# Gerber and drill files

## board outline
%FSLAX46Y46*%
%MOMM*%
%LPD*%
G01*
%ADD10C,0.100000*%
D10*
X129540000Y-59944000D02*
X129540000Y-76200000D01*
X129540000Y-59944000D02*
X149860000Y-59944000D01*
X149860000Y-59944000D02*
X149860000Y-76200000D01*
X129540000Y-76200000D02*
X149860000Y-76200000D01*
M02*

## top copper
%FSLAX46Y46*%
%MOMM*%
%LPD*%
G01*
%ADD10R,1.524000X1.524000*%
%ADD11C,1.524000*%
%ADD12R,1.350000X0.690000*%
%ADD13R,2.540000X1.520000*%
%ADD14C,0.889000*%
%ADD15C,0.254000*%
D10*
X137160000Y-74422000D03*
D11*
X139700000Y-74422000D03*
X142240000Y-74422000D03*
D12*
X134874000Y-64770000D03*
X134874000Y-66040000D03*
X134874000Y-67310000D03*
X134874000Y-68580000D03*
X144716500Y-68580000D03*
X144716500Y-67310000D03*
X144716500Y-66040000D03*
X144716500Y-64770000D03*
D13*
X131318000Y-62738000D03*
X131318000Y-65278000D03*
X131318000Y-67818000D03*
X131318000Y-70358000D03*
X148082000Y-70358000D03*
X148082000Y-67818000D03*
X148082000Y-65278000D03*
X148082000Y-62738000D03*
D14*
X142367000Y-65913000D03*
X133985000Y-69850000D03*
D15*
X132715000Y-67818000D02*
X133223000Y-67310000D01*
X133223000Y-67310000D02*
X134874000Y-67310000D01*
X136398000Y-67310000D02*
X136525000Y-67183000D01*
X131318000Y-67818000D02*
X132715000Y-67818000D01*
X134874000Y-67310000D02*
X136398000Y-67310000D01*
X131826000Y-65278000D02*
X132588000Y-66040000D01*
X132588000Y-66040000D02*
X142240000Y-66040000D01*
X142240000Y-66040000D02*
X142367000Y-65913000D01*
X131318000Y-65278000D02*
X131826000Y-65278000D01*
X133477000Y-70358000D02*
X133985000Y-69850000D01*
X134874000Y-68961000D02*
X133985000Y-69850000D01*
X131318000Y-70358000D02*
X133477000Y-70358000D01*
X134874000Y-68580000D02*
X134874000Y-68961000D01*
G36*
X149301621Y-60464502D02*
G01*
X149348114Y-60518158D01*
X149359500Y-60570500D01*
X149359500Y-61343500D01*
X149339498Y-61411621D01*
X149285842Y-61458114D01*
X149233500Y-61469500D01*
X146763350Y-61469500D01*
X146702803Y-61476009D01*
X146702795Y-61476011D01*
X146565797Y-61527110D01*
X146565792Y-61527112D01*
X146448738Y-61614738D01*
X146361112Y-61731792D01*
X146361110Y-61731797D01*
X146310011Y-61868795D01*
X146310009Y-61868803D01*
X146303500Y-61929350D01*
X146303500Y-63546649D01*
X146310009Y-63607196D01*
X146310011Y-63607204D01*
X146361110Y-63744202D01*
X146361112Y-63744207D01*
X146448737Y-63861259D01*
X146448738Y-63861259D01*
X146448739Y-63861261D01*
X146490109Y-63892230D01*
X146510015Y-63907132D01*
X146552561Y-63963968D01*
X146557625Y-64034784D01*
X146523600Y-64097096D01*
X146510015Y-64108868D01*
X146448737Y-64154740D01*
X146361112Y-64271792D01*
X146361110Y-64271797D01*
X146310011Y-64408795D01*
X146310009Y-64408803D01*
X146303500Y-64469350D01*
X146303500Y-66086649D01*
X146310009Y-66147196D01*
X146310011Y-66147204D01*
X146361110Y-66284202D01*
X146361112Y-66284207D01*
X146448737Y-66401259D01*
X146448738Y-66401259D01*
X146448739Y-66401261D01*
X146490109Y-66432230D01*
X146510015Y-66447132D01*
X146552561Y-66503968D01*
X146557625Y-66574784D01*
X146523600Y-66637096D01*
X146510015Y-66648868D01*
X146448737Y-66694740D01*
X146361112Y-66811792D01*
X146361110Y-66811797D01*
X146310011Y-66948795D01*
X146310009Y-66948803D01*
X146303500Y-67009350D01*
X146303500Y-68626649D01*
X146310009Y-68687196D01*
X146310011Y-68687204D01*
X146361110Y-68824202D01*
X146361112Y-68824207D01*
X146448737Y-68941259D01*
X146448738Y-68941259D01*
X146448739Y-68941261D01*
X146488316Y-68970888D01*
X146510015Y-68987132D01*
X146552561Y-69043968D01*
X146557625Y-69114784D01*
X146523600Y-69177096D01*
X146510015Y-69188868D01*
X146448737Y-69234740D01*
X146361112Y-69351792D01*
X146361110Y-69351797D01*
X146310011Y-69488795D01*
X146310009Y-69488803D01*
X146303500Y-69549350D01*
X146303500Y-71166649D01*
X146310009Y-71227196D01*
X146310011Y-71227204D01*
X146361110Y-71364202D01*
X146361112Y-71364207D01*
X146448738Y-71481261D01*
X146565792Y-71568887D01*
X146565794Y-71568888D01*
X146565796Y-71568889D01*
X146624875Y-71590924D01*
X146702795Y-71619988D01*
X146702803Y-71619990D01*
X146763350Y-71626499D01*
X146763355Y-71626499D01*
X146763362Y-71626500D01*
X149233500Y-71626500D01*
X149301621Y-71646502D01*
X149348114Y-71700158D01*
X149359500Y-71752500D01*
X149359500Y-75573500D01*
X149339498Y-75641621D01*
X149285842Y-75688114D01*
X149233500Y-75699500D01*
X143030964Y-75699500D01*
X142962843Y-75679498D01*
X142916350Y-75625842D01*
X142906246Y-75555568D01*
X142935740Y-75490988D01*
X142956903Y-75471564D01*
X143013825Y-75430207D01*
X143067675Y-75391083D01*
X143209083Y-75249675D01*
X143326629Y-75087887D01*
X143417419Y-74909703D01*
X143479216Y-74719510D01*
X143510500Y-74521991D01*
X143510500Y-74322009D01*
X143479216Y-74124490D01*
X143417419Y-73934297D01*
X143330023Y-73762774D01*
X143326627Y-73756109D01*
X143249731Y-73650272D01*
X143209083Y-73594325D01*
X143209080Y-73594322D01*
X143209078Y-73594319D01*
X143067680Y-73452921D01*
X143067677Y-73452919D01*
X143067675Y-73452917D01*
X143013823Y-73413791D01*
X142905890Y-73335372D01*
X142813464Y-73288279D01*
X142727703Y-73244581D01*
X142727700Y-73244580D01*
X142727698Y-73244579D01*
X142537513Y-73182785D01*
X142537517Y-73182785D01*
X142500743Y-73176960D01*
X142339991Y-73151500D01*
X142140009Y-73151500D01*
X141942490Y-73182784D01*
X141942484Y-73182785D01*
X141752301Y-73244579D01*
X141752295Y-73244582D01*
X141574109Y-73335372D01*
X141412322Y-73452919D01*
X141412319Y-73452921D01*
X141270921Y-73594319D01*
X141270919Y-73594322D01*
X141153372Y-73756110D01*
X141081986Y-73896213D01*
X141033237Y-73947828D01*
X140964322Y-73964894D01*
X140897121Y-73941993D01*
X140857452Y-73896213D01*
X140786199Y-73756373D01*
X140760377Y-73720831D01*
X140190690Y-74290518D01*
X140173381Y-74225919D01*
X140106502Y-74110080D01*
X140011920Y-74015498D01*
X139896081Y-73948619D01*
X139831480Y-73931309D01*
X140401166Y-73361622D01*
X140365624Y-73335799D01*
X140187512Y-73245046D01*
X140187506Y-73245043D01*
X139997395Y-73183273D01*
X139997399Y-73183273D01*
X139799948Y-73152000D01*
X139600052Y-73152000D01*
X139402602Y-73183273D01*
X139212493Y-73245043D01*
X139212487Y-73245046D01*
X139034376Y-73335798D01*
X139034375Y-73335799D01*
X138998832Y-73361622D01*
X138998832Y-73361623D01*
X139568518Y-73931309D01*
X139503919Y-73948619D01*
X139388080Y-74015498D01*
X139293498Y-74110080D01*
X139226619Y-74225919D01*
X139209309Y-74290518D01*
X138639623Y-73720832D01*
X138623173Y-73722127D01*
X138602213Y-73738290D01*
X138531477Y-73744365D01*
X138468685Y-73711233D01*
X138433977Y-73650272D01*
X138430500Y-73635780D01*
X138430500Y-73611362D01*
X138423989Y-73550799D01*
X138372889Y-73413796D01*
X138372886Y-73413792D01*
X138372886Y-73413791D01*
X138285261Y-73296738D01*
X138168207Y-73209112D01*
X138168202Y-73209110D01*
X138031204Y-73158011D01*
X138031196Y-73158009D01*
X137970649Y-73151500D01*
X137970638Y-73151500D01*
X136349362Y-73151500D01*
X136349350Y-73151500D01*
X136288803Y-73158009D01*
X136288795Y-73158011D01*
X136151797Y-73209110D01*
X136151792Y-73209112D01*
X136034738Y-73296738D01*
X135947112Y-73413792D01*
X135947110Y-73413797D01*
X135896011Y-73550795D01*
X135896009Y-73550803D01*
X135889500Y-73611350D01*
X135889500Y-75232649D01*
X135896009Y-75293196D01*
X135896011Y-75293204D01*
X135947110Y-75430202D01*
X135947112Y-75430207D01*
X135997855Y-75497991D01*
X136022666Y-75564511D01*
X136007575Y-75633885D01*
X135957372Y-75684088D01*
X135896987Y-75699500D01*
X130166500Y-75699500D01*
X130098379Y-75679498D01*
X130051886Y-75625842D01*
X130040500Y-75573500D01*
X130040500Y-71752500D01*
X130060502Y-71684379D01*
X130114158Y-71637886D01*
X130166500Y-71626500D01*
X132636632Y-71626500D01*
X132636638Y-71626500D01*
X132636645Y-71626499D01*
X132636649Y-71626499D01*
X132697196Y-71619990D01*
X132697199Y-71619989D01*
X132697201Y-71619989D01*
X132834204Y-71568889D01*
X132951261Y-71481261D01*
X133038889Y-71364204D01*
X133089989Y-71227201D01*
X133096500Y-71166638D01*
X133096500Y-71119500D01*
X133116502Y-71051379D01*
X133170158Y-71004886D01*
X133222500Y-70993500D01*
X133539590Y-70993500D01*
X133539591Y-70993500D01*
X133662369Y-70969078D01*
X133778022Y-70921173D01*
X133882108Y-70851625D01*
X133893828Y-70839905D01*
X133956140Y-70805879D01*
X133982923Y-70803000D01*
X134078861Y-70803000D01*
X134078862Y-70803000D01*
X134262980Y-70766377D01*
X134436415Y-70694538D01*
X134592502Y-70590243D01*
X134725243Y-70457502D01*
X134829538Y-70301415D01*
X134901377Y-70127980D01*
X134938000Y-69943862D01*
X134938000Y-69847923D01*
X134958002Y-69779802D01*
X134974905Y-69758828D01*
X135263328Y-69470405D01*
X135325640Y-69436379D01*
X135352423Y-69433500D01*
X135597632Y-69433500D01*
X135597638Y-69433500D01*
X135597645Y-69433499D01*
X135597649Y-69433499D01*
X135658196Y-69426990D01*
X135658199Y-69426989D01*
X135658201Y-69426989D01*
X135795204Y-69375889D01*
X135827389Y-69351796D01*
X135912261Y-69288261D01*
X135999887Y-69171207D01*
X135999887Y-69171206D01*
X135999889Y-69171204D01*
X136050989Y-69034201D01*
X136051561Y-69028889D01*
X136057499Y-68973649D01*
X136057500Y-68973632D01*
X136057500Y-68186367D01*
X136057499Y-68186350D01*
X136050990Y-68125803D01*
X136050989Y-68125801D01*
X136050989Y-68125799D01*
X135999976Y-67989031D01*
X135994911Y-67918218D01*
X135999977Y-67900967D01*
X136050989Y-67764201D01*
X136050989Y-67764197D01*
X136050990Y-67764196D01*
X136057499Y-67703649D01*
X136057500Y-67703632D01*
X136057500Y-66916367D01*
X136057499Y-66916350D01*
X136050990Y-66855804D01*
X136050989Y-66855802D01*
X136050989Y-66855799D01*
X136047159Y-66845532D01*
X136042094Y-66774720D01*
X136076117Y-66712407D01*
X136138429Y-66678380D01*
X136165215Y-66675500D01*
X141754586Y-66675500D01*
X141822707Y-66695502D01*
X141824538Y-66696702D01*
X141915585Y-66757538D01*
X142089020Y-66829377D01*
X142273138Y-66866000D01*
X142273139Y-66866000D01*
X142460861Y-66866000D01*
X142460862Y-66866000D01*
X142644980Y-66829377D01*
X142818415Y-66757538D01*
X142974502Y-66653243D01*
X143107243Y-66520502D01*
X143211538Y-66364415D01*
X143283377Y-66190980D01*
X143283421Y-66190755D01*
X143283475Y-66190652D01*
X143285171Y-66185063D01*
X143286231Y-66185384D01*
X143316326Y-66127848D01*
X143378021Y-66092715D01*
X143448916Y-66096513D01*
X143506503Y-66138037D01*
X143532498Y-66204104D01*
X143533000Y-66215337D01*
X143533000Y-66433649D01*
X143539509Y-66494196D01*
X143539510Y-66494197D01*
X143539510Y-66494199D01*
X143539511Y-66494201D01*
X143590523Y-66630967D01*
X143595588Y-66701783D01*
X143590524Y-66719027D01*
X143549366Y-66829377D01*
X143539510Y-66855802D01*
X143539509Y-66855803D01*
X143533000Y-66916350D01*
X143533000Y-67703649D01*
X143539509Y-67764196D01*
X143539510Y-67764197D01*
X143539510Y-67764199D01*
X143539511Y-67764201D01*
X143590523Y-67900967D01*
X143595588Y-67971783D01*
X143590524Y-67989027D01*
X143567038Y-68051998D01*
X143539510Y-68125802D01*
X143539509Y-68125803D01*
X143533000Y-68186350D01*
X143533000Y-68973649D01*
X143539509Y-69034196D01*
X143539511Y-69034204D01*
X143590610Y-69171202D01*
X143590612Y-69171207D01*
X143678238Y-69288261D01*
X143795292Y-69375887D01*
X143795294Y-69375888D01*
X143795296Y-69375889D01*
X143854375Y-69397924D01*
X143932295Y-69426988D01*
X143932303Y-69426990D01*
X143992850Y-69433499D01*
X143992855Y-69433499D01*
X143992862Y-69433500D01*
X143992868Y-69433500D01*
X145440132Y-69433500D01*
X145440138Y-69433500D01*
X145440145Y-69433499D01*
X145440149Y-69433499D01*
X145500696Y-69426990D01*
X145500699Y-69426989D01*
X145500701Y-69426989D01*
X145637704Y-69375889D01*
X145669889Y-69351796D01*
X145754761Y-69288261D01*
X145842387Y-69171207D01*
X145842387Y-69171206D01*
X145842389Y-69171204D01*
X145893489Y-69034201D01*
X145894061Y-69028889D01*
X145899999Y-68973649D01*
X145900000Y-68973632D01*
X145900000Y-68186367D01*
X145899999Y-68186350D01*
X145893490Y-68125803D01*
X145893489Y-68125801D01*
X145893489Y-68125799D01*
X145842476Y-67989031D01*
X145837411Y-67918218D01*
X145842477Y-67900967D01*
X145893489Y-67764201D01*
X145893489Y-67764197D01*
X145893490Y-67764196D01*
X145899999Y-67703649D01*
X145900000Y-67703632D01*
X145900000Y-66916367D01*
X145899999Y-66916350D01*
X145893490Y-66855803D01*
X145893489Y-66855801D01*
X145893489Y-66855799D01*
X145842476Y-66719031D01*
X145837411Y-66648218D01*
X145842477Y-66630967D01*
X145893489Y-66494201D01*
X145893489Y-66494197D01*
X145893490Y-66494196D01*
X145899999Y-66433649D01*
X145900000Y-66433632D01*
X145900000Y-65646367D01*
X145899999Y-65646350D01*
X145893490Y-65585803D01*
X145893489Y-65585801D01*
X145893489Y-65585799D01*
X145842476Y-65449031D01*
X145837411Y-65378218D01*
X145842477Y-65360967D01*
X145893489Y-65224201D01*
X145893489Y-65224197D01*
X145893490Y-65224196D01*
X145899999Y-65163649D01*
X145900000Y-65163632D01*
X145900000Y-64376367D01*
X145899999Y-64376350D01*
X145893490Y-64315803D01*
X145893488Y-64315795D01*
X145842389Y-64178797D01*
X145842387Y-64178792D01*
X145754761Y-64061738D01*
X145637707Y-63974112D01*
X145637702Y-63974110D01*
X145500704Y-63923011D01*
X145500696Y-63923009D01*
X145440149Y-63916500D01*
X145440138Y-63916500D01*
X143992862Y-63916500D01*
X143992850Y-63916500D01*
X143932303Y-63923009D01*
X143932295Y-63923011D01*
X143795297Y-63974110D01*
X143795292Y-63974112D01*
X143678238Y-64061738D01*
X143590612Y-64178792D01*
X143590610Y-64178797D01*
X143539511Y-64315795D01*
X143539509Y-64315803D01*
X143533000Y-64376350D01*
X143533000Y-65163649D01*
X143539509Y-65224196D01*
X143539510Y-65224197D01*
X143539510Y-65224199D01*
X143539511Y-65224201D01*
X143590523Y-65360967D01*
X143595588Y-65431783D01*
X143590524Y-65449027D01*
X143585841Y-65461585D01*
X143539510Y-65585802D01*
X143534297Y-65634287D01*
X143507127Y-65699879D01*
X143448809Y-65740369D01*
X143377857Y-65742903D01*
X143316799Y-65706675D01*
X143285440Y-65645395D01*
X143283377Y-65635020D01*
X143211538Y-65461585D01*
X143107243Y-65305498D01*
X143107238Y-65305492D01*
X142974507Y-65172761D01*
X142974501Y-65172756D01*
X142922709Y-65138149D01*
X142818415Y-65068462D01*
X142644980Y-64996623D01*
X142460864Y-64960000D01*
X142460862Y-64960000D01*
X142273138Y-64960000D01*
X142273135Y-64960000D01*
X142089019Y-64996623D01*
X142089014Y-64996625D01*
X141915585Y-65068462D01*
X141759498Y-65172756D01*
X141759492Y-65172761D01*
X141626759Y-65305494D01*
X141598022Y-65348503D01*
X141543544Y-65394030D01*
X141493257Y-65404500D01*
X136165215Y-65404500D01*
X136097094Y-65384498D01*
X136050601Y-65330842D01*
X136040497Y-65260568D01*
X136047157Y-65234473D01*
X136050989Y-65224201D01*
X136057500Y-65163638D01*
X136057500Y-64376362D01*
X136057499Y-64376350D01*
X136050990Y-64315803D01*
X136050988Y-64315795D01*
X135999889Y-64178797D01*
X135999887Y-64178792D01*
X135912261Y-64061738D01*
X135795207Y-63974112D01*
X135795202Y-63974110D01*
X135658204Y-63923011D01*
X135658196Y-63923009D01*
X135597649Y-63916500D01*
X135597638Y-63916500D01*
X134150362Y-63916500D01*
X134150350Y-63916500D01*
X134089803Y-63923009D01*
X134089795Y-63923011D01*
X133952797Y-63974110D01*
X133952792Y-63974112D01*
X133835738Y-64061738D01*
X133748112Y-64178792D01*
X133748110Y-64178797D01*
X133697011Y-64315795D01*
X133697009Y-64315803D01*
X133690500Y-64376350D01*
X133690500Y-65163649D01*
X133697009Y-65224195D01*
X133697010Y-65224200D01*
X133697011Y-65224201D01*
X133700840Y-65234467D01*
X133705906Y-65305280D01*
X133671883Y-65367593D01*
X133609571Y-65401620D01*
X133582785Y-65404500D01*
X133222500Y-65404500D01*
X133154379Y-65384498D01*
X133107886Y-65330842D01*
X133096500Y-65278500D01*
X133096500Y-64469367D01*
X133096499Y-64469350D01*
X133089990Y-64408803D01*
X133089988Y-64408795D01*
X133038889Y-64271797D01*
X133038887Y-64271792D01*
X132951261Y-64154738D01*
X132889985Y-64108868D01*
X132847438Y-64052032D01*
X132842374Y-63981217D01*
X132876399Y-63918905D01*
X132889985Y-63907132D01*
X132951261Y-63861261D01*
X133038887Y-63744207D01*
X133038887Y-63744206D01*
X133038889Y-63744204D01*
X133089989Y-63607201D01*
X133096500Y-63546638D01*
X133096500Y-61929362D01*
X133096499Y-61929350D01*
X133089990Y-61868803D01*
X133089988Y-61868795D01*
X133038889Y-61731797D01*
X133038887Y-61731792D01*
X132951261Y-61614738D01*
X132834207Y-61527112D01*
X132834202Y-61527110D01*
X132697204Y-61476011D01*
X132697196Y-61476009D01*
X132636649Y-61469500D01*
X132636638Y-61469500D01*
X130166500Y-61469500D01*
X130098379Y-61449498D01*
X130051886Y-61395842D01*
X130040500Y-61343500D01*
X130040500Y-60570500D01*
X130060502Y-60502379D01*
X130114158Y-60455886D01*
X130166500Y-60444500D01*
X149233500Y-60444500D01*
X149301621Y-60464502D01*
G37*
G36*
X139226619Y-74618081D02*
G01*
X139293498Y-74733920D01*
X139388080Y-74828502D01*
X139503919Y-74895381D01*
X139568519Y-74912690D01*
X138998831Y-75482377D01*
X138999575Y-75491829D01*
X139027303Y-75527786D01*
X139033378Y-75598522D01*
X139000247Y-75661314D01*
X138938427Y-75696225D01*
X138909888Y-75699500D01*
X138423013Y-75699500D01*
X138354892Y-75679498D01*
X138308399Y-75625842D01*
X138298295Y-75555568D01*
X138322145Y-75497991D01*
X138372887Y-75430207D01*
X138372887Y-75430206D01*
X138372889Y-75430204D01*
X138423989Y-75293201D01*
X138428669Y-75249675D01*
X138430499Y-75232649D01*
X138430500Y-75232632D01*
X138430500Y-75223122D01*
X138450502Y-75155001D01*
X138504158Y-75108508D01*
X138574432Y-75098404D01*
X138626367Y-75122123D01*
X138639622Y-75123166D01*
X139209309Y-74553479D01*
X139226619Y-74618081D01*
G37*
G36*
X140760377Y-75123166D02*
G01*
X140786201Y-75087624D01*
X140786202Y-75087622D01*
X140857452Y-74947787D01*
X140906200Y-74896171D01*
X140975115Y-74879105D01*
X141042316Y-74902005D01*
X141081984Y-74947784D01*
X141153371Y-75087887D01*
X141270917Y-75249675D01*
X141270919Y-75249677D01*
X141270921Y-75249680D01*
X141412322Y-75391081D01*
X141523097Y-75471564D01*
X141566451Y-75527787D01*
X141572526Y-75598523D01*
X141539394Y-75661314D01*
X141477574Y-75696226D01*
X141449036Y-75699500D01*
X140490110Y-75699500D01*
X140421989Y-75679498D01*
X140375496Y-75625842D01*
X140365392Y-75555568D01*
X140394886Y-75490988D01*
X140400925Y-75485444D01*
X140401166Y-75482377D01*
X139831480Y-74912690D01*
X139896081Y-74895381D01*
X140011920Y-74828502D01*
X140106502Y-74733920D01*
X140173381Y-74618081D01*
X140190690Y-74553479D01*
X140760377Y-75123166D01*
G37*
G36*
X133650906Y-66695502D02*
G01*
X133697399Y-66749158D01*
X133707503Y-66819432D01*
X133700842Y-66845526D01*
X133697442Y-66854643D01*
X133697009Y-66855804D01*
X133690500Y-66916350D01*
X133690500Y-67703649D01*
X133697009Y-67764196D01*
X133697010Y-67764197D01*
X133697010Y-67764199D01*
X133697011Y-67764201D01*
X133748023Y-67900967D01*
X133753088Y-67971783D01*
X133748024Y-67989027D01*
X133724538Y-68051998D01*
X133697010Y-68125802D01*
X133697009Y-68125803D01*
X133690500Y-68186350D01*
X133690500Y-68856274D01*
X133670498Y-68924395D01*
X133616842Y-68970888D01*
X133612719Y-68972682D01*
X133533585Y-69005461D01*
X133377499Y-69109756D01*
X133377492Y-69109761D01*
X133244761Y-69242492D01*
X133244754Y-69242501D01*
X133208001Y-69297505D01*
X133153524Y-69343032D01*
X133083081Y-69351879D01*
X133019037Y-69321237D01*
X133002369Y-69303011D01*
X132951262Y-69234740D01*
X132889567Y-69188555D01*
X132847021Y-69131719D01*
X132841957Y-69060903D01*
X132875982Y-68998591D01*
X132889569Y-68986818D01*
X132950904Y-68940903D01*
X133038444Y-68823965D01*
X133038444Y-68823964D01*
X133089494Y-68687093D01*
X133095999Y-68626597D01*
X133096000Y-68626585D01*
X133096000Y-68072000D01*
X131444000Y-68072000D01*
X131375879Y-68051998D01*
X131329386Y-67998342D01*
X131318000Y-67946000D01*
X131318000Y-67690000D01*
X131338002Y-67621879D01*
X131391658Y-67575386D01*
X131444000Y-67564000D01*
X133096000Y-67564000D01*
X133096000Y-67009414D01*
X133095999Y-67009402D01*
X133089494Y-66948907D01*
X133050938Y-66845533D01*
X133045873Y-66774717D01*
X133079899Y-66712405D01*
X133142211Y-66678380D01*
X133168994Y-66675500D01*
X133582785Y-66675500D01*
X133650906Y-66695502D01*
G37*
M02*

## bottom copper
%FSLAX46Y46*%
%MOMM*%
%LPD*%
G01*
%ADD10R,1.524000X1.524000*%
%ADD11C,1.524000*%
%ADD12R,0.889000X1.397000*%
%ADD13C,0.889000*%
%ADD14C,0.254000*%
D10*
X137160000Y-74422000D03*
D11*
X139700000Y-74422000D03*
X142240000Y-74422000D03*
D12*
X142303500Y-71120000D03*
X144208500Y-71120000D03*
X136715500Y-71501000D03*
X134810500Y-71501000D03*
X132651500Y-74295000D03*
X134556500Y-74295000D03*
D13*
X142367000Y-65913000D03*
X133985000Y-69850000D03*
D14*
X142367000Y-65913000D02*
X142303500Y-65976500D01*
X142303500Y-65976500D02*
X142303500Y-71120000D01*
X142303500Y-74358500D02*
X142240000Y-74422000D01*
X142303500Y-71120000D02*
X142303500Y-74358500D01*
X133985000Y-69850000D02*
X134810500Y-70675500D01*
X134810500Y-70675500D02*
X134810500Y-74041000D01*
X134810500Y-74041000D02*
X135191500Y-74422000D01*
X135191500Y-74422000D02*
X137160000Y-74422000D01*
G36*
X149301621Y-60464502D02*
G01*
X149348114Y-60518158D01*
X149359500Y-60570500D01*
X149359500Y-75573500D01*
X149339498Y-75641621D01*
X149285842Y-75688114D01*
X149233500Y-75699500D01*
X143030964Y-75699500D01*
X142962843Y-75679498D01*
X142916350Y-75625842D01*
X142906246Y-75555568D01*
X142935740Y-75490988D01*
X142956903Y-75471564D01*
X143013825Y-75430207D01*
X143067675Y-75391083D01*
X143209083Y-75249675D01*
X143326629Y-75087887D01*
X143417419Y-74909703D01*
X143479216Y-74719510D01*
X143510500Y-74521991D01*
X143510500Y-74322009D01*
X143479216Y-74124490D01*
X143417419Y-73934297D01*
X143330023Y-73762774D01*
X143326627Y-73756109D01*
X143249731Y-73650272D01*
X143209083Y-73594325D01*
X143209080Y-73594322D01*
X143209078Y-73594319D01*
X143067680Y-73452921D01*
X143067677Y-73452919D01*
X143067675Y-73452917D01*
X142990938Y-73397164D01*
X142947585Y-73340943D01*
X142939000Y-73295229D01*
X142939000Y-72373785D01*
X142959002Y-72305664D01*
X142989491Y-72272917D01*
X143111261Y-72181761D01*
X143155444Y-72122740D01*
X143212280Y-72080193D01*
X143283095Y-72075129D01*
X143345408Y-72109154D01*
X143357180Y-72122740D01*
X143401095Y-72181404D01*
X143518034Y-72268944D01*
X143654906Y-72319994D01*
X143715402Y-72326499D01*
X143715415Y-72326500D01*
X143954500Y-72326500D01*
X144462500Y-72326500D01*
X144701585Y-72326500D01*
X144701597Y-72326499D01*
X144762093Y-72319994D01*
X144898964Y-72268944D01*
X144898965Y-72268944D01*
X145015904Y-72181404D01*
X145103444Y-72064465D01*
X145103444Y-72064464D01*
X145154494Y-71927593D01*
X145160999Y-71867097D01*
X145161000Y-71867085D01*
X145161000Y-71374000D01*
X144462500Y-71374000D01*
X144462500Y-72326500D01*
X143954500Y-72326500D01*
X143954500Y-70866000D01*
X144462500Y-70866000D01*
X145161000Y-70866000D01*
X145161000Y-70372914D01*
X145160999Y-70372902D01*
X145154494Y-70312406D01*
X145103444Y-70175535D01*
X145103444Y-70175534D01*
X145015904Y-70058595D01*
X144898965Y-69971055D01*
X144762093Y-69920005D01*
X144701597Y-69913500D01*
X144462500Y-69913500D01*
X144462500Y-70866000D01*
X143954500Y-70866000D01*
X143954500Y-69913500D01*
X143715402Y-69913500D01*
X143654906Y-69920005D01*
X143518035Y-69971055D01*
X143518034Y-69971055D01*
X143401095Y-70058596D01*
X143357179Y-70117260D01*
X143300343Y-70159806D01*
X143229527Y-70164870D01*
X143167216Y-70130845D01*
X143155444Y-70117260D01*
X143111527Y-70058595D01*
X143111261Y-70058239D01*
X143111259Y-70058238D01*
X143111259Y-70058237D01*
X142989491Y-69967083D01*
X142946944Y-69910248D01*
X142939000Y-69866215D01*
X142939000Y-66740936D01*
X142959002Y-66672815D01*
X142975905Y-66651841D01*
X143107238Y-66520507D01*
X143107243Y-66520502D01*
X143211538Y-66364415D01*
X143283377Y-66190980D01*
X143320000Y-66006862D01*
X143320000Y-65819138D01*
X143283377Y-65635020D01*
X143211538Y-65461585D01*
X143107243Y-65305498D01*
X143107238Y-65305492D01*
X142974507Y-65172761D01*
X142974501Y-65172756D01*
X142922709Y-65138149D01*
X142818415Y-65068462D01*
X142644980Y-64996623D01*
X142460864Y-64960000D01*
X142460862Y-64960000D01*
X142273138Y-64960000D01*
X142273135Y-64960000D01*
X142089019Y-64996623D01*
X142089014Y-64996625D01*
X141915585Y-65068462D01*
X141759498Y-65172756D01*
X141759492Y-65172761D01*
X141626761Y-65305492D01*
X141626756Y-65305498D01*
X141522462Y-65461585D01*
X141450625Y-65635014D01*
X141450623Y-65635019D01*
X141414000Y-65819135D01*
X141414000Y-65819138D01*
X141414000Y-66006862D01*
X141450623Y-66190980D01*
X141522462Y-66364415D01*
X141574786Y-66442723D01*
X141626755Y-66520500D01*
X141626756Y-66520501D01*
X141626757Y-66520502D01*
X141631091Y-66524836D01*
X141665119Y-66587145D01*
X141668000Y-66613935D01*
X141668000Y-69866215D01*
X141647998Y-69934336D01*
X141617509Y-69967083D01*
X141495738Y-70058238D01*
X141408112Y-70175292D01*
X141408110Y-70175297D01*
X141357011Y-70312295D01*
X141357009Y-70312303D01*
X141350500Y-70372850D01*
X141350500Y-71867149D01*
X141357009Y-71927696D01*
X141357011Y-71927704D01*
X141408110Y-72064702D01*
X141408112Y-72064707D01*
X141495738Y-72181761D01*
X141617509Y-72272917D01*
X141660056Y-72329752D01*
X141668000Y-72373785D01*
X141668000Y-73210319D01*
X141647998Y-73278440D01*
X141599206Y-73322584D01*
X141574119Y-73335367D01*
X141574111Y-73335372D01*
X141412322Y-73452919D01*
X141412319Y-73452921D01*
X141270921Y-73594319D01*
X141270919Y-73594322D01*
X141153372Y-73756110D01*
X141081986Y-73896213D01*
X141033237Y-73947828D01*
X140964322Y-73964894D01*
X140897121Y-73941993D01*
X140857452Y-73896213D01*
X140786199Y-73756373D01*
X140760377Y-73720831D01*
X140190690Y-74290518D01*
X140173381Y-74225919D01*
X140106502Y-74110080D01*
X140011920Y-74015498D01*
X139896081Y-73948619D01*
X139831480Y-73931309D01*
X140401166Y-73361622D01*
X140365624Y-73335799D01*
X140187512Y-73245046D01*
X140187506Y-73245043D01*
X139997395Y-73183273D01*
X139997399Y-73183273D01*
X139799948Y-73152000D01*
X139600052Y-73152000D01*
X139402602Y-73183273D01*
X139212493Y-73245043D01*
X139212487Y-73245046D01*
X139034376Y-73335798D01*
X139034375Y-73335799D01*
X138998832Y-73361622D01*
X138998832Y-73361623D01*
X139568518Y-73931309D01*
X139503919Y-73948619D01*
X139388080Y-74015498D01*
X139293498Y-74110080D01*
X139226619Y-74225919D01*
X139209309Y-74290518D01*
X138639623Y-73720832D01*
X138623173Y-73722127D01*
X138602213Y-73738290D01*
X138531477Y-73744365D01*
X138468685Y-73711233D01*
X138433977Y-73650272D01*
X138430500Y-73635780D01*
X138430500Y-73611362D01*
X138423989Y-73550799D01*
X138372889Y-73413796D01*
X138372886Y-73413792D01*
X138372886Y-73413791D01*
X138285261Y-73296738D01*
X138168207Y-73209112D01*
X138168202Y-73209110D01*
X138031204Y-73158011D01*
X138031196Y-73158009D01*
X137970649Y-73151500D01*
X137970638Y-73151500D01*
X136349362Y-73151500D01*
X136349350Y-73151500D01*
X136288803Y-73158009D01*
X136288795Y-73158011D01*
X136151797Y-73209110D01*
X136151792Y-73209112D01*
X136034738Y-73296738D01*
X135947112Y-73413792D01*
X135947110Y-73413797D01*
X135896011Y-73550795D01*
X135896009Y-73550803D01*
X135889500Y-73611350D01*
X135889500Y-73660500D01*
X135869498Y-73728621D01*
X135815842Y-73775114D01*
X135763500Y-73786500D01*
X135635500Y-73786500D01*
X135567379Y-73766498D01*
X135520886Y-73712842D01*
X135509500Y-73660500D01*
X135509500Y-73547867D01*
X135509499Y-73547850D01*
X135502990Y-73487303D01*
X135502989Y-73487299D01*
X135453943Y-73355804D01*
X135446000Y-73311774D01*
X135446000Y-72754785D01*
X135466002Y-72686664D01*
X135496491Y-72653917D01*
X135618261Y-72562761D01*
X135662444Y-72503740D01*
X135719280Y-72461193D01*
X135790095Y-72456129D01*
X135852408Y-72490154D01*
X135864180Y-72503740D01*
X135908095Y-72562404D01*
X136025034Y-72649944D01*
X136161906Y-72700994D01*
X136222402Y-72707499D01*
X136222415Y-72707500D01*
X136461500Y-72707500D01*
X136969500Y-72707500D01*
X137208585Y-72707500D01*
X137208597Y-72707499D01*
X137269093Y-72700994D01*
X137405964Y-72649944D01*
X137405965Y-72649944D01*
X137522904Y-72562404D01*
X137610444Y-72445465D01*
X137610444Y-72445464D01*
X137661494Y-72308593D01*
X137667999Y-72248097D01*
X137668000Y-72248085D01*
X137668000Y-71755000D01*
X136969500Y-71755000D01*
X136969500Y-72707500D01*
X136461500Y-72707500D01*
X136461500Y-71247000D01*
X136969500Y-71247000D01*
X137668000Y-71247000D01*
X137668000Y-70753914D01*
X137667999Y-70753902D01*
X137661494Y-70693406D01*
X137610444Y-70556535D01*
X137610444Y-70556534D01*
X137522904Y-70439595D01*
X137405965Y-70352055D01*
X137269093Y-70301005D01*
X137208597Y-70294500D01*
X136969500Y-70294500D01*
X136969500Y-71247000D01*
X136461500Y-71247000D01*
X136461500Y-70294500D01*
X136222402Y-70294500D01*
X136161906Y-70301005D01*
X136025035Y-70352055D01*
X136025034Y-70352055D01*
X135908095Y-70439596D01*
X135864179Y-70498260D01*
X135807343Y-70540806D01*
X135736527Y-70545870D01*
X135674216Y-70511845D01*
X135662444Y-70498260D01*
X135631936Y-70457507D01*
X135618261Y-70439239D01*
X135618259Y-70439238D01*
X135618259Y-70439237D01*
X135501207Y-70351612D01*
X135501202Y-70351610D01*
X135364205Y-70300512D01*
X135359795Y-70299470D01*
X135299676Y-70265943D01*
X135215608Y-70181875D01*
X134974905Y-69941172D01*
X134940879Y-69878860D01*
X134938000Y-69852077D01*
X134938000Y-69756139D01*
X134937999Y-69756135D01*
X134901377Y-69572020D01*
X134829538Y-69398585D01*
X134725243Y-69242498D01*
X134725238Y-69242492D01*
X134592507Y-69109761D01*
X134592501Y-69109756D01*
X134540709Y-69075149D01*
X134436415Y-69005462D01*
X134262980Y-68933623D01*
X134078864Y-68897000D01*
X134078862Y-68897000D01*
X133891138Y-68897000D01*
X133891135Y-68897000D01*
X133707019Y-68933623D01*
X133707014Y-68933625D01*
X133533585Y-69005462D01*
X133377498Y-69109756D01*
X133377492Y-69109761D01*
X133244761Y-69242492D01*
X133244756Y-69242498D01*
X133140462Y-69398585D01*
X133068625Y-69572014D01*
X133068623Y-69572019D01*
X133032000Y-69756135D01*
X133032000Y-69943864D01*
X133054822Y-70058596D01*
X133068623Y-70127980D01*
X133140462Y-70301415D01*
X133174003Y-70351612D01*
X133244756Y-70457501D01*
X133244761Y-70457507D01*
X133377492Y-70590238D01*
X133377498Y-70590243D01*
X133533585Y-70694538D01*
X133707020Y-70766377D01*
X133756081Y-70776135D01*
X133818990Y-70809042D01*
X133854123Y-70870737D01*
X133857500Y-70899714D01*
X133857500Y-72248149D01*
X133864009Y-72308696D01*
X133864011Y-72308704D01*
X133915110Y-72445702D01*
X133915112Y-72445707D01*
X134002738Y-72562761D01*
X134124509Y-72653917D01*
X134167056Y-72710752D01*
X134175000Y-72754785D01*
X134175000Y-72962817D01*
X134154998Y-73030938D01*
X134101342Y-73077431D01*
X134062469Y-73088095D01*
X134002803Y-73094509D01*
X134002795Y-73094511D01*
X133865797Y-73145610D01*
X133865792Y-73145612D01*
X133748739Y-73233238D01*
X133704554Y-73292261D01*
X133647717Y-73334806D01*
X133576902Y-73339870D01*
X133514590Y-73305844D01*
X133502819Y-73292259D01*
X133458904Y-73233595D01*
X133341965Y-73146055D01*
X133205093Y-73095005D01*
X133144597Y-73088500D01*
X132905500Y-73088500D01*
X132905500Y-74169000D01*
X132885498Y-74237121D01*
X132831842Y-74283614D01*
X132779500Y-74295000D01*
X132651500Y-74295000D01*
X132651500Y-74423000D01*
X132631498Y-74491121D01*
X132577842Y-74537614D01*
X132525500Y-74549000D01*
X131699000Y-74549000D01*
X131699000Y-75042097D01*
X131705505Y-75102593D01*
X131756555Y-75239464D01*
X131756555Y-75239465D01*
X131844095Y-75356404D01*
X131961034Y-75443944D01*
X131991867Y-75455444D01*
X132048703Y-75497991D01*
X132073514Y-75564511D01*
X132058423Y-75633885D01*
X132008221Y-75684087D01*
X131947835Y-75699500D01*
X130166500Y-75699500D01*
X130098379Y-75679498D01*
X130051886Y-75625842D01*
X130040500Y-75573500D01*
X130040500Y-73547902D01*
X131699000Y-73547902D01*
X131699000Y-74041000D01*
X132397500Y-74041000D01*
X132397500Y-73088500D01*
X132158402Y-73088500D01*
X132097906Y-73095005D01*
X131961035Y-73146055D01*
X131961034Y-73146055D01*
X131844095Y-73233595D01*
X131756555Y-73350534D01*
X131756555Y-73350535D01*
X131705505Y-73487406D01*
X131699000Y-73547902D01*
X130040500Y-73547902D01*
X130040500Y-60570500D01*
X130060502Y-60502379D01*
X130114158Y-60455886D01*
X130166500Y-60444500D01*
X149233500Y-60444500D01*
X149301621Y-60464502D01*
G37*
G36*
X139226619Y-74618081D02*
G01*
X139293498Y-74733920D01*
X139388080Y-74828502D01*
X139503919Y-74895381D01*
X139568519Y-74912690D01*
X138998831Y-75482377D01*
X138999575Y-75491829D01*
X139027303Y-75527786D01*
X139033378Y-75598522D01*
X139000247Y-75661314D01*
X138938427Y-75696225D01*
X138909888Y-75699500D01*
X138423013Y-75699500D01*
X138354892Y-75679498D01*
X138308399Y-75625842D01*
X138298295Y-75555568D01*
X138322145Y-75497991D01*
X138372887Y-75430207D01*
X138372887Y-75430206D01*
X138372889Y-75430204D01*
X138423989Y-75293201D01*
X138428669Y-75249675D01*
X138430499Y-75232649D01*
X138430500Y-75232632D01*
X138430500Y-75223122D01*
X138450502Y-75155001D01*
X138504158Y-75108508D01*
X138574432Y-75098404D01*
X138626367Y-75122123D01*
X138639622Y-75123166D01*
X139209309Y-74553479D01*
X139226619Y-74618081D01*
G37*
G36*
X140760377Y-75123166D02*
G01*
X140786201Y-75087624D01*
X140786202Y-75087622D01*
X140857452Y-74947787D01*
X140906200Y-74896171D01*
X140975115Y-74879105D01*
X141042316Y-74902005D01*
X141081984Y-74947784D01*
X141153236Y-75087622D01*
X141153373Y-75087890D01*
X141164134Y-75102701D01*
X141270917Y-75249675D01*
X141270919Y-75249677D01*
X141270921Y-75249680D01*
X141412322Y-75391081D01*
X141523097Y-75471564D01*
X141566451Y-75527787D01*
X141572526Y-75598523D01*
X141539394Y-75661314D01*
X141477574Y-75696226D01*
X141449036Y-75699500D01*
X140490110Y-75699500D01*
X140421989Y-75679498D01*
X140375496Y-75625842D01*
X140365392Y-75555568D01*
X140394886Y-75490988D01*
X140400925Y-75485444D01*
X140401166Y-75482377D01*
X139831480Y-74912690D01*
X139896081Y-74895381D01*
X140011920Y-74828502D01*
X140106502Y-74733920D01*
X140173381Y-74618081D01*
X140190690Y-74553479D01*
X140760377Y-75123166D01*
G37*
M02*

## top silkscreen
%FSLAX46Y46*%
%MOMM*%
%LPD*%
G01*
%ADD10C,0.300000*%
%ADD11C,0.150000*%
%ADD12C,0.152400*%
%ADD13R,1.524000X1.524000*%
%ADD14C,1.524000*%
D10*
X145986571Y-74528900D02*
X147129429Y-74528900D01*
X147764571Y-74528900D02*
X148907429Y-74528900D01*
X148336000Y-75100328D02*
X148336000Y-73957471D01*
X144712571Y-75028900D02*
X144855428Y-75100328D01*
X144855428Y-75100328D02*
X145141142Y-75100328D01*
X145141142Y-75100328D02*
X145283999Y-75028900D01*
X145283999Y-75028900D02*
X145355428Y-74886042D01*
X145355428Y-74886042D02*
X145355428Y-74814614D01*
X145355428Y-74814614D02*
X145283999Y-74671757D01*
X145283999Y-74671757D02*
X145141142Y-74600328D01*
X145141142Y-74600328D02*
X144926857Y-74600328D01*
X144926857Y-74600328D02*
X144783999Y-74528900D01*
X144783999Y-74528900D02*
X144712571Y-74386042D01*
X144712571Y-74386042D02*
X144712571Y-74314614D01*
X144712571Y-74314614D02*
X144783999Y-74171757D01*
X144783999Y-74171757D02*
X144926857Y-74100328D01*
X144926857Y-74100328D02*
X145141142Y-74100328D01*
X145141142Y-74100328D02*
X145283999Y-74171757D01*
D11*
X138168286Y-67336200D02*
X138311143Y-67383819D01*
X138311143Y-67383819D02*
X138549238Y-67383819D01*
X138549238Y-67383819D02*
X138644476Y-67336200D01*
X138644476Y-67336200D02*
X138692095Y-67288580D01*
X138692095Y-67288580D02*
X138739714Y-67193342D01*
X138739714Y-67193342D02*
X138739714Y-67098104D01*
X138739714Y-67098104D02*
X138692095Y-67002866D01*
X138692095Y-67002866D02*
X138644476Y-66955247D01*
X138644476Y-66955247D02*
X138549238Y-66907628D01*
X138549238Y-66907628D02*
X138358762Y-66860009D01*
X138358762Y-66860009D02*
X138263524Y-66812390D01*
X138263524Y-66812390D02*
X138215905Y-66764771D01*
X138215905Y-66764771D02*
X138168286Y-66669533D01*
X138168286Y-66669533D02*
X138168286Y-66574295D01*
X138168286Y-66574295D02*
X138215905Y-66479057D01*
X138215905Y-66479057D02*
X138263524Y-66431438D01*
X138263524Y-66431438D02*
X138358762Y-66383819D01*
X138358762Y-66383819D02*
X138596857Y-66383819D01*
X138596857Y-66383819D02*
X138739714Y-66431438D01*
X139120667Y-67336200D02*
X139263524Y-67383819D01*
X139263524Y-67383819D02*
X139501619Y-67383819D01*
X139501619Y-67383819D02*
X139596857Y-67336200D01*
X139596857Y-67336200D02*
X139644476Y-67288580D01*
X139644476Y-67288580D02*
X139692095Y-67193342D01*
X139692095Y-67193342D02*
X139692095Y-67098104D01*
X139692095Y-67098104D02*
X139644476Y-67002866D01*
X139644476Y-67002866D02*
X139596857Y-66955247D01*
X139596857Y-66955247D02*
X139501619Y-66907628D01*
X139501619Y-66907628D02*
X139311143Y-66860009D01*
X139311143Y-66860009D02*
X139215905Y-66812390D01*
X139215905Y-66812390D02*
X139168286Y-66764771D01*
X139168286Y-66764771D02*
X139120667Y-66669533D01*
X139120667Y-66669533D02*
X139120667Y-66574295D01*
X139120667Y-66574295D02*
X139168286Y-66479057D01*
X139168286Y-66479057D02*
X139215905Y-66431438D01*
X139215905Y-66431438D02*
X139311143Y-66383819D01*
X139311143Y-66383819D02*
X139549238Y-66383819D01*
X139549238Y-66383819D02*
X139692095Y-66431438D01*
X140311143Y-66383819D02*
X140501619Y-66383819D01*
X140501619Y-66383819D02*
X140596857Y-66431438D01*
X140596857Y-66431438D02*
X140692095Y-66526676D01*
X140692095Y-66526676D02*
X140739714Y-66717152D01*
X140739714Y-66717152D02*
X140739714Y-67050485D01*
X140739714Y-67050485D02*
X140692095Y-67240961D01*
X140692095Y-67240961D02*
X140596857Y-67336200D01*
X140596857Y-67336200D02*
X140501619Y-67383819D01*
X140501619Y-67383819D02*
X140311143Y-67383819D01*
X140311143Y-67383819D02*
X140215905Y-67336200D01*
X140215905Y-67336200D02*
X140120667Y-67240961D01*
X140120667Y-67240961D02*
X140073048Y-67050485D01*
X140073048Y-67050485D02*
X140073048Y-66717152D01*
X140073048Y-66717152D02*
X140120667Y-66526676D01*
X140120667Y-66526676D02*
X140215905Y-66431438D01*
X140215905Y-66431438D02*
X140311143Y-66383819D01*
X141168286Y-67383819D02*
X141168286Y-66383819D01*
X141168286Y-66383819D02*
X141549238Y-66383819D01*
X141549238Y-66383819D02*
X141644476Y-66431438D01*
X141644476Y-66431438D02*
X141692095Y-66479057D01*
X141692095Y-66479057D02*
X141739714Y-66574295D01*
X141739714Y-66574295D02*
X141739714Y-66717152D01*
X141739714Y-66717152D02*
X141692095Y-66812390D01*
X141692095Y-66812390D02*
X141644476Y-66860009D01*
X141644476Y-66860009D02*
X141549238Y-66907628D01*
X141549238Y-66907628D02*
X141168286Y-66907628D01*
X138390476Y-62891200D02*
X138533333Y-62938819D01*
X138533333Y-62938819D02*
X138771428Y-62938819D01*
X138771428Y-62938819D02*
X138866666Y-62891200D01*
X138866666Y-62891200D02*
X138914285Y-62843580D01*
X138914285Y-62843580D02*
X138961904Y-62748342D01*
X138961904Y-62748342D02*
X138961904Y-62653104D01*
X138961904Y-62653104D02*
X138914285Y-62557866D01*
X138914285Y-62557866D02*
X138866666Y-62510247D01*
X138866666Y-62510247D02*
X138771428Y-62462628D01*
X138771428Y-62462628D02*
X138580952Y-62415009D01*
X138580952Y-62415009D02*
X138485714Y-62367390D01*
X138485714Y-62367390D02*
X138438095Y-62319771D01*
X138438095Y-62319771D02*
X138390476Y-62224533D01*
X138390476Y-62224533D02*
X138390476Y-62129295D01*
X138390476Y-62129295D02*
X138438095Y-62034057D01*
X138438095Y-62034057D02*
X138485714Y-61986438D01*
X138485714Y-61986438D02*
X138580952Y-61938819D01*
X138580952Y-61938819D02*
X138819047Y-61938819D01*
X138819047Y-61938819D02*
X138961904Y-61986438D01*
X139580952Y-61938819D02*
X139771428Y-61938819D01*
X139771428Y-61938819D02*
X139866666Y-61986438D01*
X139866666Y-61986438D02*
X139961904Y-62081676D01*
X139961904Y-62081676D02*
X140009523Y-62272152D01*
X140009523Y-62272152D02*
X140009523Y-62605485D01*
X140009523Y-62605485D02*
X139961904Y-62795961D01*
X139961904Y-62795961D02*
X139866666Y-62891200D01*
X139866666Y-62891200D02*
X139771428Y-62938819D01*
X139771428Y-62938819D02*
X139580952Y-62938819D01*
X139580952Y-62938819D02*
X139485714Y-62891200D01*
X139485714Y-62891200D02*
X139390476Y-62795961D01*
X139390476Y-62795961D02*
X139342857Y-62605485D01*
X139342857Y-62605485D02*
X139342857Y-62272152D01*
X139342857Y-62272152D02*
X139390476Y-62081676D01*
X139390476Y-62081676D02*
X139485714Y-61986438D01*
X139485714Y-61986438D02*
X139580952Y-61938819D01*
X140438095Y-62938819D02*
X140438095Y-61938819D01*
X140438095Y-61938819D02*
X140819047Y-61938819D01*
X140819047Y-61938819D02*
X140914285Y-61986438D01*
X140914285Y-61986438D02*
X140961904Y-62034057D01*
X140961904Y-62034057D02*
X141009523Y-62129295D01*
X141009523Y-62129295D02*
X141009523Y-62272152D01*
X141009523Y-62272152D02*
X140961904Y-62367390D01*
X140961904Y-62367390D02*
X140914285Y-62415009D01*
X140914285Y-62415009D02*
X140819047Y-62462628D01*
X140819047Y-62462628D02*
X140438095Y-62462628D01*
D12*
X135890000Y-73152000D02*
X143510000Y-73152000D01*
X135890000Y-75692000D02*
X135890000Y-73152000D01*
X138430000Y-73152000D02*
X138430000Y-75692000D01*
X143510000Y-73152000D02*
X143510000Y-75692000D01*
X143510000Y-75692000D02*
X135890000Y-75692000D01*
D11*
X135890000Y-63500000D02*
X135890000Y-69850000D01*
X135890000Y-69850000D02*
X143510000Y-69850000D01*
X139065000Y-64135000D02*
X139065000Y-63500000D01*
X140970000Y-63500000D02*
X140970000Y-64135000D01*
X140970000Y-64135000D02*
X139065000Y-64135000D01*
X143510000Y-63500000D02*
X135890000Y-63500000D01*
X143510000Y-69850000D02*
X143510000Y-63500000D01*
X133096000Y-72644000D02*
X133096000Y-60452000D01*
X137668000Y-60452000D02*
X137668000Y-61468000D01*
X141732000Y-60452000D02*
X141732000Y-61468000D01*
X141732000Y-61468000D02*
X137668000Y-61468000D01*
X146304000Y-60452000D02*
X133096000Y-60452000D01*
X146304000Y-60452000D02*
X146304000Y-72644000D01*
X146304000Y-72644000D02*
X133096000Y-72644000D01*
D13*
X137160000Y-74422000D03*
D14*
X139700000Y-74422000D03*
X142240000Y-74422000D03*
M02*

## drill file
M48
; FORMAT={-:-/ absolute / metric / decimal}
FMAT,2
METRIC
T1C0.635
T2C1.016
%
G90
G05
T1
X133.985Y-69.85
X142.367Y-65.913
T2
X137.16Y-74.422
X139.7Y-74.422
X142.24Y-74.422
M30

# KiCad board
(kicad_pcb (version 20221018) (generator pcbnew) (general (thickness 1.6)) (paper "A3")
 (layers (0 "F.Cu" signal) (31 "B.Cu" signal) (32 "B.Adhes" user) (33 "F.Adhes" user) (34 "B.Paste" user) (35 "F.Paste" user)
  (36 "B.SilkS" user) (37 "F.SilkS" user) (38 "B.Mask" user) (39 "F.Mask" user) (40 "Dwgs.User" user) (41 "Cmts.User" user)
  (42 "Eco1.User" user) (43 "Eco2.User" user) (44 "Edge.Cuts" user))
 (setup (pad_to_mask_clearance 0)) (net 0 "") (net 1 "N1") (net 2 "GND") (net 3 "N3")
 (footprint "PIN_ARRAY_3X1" (layer "F.Cu") (at 139.7 74.422)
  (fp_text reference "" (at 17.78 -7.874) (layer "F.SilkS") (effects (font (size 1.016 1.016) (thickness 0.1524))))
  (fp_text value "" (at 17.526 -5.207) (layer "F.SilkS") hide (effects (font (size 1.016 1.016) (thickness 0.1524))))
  (fp_line (start -3.81 -1.27) (end 3.81 -1.27) (stroke (width 0.1524) (type solid)) (layer "F.SilkS"))
  (fp_line (start -3.81 1.27) (end -3.81 -1.27) (stroke (width 0.1524) (type solid)) (layer "F.SilkS"))
  (fp_line (start -1.27 -1.27) (end -1.27 1.27) (stroke (width 0.1524) (type solid)) (layer "F.SilkS"))
  (fp_line (start 3.81 -1.27) (end 3.81 1.27) (stroke (width 0.1524) (type solid)) (layer "F.SilkS"))
  (fp_line (start 3.81 1.27) (end -3.81 1.27) (stroke (width 0.1524) (type solid)) (layer "F.SilkS"))
  (pad "1" thru_hole rect (at -2.54 0) (size 1.524 1.524) (drill 1.016) (layers "*.Cu" "*.Mask" "F.SilkS") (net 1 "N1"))
  (pad "2" thru_hole circle (at 0 0) (size 1.524 1.524) (drill 1.016) (layers "*.Cu" "*.Mask" "F.SilkS") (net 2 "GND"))
  (pad "3" thru_hole circle (at 2.54 0) (size 1.524 1.524) (drill 1.016) (layers "*.Cu" "*.Mask" "F.SilkS") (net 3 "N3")))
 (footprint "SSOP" (layer "F.Cu") (at 139.7 66.675)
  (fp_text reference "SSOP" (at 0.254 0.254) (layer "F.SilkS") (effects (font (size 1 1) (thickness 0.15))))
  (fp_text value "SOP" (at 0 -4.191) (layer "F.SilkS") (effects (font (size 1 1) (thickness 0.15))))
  (fp_line (start -3.81 -3.175) (end -3.81 3.175) (stroke (width 0.15) (type solid)) (layer "F.SilkS"))
  (fp_line (start -3.81 3.175) (end 3.81 3.175) (stroke (width 0.15) (type solid)) (layer "F.SilkS"))
  (fp_line (start -0.635 -2.54) (end -0.635 -3.175) (stroke (width 0.15) (type solid)) (layer "F.SilkS"))
  (fp_line (start 1.27 -3.175) (end 1.27 -2.54) (stroke (width 0.15) (type solid)) (layer "F.SilkS"))
  (fp_line (start 1.27 -2.54) (end -0.635 -2.54) (stroke (width 0.15) (type solid)) (layer "F.SilkS"))
  (fp_line (start 3.81 -3.175) (end -3.81 -3.175) (stroke (width 0.15) (type solid)) (layer "F.SilkS"))
  (fp_line (start 3.81 3.175) (end 3.81 -3.175) (stroke (width 0.15) (type solid)) (layer "F.SilkS"))
  (pad "1" smd rect (at -4.826 -1.905 270) (size 0.69 1.35) (layers "F.Cu" "F.Paste" "F.Mask"))
  (pad "2" smd rect (at -4.826 -0.635 270) (size 0.69 1.35) (layers "F.Cu" "F.Paste" "F.Mask"))
  (pad "3" smd rect (at -4.826 0.635 270) (size 0.69 1.35) (layers "F.Cu" "F.Paste" "F.Mask"))
  (pad "4" smd rect (at -4.826 1.905 270) (size 0.69 1.35) (layers "F.Cu" "F.Paste" "F.Mask"))
  (pad "5" smd rect (at 5.0165 1.905 270) (size 0.69 1.35) (layers "F.Cu" "F.Paste" "F.Mask"))
  (pad "6" smd rect (at 5.0165 0.635 270) (size 0.69 1.35) (layers "F.Cu" "F.Paste" "F.Mask"))
  (pad "7" smd rect (at 5.0165 -0.635 270) (size 0.69 1.35) (layers "F.Cu" "F.Paste" "F.Mask"))
  (pad "8" smd rect (at 5.0165 -1.905 270) (size 0.69 1.35) (layers "F.Cu" "F.Paste" "F.Mask")))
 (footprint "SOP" (layer "F.Cu") (at 139.7 66.548)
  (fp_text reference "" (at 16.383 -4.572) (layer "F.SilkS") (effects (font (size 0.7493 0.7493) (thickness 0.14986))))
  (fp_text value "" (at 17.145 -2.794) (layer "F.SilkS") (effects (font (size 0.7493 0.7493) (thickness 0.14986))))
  (fp_line (start -6.604 6.096) (end -6.604 -6.096) (stroke (width 0.15) (type solid)) (layer "F.SilkS"))
  (fp_line (start -2.032 -6.096) (end -2.032 -5.08) (stroke (width 0.15) (type solid)) (layer "F.SilkS"))
  (fp_line (start 2.032 -6.096) (end 2.032 -5.08) (stroke (width 0.15) (type solid)) (layer "F.SilkS"))
  (fp_line (start 2.032 -5.08) (end -2.032 -5.08) (stroke (width 0.15) (type solid)) (layer "F.SilkS"))
  (fp_line (start 6.604 -6.096) (end -6.604 -6.096) (stroke (width 0.15) (type solid)) (layer "F.SilkS"))
  (fp_line (start 6.604 -6.096) (end 6.604 6.096) (stroke (width 0.15) (type solid)) (layer "F.SilkS"))
  (fp_line (start 6.604 6.096) (end -6.604 6.096) (stroke (width 0.15) (type solid)) (layer "F.SilkS"))
  (pad "1" smd rect (at -8.382 -3.81 270) (size 1.52 2.54) (layers "F.Cu" "F.Paste" "F.Mask"))
  (pad "2" smd rect (at -8.382 -1.27 270) (size 1.52 2.54) (layers "F.Cu" "F.Paste" "F.Mask") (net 3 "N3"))
  (pad "3" smd rect (at -8.382 1.27 270) (size 1.52 2.54) (layers "F.Cu" "F.Paste" "F.Mask") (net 2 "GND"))
  (pad "4" smd rect (at -8.382 3.81 270) (size 1.52 2.54) (layers "F.Cu" "F.Paste" "F.Mask") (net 1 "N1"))
  (pad "5" smd rect (at 8.382 3.81 270) (size 1.52 2.54) (layers "F.Cu" "F.Paste" "F.Mask"))
  (pad "6" smd rect (at 8.382 1.27 270) (size 1.52 2.54) (layers "F.Cu" "F.Paste" "F.Mask"))
  (pad "7" smd rect (at 8.382 -1.27 270) (size 1.52 2.54) (layers "F.Cu" "F.Paste" "F.Mask"))
  (pad "8" smd rect (at 8.382 -3.81 270) (size 1.52 2.54) (layers "F.Cu" "F.Paste" "F.Mask")))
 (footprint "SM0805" (layer "B.Cu") (at 143.256 71.12)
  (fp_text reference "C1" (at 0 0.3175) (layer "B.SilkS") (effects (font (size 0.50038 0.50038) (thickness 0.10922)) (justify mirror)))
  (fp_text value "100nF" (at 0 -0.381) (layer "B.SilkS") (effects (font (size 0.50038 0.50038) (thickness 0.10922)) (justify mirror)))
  (pad "1" smd rect (at -0.9525 0) (size 0.889 1.397) (layers "B.Cu" "B.Paste" "B.Mask") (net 3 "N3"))
  (pad "2" smd rect (at 0.9525 0) (size 0.889 1.397) (layers "B.Cu" "B.Paste" "B.Mask") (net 2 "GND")))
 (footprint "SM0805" (layer "B.Cu") (at 135.763 71.501 180)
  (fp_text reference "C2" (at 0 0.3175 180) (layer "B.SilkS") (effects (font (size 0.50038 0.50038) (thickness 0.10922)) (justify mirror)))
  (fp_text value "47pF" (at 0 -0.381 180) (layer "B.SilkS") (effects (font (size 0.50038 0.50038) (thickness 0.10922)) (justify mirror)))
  (pad "1" smd rect (at -0.9525 0 180) (size 0.889 1.397) (layers "B.Cu" "B.Paste" "B.Mask") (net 2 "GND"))
  (pad "2" smd rect (at 0.9525 0 180) (size 0.889 1.397) (layers "B.Cu" "B.Paste" "B.Mask") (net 1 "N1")))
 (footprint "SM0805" (layer "B.Cu") (at 133.604 74.295)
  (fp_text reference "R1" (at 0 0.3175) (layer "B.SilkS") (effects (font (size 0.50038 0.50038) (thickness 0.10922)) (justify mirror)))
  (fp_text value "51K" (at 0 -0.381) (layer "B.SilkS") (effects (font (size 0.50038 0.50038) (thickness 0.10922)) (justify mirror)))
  (pad "1" smd rect (at -0.9525 0) (size 0.889 1.397) (layers "B.Cu" "B.Paste" "B.Mask") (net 2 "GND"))
  (pad "2" smd rect (at 0.9525 0) (size 0.889 1.397) (layers "B.Cu" "B.Paste" "B.Mask") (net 1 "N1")))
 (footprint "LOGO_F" (layer "B.Cu") (at 146.177 66.675)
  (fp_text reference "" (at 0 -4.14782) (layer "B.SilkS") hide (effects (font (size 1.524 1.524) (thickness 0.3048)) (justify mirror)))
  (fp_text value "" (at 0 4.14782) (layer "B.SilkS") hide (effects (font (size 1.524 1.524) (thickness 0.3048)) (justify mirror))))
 (gr_line (start 129.54 59.944) (end 129.54 76.2) (stroke (width 0.1) (type solid)) (layer "Edge.Cuts"))
 (gr_line (start 129.54 59.944) (end 149.86 59.944) (stroke (width 0.1) (type solid)) (layer "Edge.Cuts"))
 (gr_line (start 149.86 59.944) (end 149.86 76.2) (stroke (width 0.1) (type solid)) (layer "Edge.Cuts"))
 (gr_line (start 129.54 76.2) (end 149.86 76.2) (stroke (width 0.1) (type solid)) (layer "Edge.Cuts"))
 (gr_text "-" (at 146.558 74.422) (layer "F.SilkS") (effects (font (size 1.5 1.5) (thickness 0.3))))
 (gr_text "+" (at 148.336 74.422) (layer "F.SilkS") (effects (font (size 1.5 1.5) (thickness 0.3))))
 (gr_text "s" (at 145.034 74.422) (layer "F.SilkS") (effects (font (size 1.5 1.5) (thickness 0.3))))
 (segment (start 132.715 67.818) (end 133.223 67.31) (width 0.254) (layer "F.Cu") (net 2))
 (segment (start 133.223 67.31) (end 134.874 67.31) (width 0.254) (layer "F.Cu") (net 2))
 (segment (start 136.398 67.31) (end 136.525 67.183) (width 0.254) (layer "F.Cu") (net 2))
 (segment (start 131.318 67.818) (end 132.715 67.818) (width 0.254) (layer "F.Cu") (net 2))
 (segment (start 134.874 67.31) (end 136.398 67.31) (width 0.254) (layer "F.Cu") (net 2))
 (segment (start 131.826 65.278) (end 132.588 66.04) (width 0.254) (layer "F.Cu") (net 3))
 (segment (start 132.588 66.04) (end 142.24 66.04) (width 0.254) (layer "F.Cu") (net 3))
 (segment (start 142.24 66.04) (end 142.367 65.913) (width 0.254) (layer "F.Cu") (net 3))
 (segment (start 131.318 65.278) (end 131.826 65.278) (width 0.254) (layer "F.Cu") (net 3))
 (via (at 142.367 65.913) (size 0.889) (drill 0.635) (layers "F.Cu" "B.Cu") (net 3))
 (segment (start 142.367 65.913) (end 142.3035 65.9765) (width 0.254) (layer "B.Cu") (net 3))
 (segment (start 142.3035 65.9765) (end 142.3035 71.12) (width 0.254) (layer "B.Cu") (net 3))
 (segment (start 142.3035 74.3585) (end 142.24 74.422) (width 0.254) (layer "B.Cu") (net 3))
 (segment (start 142.3035 71.12) (end 142.3035 74.3585) (width 0.254) (layer "B.Cu") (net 3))
 (segment (start 133.477 70.358) (end 133.985 69.85) (width 0.254) (layer "F.Cu") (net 1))
 (segment (start 134.874 68.961) (end 133.985 69.85) (width 0.254) (layer "F.Cu") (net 1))
 (segment (start 131.318 70.358) (end 133.477 70.358) (width 0.254) (layer "F.Cu") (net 1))
 (segment (start 134.874 68.58) (end 134.874 68.961) (width 0.254) (layer "F.Cu") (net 1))
 (via (at 133.985 69.85) (size 0.889) (drill 0.635) (layers "F.Cu" "B.Cu") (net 1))
 (segment (start 133.985 69.85) (end 134.8105 70.6755) (width 0.254) (layer "B.Cu") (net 1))
 (segment (start 134.8105 70.6755) (end 134.8105 74.041) (width 0.254) (layer "B.Cu") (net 1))
 (segment (start 134.8105 74.041) (end 135.1915 74.422) (width 0.254) (layer "B.Cu") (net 1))
 (segment (start 135.1915 74.422) (end 137.16 74.422) (width 0.254) (layer "B.Cu") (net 1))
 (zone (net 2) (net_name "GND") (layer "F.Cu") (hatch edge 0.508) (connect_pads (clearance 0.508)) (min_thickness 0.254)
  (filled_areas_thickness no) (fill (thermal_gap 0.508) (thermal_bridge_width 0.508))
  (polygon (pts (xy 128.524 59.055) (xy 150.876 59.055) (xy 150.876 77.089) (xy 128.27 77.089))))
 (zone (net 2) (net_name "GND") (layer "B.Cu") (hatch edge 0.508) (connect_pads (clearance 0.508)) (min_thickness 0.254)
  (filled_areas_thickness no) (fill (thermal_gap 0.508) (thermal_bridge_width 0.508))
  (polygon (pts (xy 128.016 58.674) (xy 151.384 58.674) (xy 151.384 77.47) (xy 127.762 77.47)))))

